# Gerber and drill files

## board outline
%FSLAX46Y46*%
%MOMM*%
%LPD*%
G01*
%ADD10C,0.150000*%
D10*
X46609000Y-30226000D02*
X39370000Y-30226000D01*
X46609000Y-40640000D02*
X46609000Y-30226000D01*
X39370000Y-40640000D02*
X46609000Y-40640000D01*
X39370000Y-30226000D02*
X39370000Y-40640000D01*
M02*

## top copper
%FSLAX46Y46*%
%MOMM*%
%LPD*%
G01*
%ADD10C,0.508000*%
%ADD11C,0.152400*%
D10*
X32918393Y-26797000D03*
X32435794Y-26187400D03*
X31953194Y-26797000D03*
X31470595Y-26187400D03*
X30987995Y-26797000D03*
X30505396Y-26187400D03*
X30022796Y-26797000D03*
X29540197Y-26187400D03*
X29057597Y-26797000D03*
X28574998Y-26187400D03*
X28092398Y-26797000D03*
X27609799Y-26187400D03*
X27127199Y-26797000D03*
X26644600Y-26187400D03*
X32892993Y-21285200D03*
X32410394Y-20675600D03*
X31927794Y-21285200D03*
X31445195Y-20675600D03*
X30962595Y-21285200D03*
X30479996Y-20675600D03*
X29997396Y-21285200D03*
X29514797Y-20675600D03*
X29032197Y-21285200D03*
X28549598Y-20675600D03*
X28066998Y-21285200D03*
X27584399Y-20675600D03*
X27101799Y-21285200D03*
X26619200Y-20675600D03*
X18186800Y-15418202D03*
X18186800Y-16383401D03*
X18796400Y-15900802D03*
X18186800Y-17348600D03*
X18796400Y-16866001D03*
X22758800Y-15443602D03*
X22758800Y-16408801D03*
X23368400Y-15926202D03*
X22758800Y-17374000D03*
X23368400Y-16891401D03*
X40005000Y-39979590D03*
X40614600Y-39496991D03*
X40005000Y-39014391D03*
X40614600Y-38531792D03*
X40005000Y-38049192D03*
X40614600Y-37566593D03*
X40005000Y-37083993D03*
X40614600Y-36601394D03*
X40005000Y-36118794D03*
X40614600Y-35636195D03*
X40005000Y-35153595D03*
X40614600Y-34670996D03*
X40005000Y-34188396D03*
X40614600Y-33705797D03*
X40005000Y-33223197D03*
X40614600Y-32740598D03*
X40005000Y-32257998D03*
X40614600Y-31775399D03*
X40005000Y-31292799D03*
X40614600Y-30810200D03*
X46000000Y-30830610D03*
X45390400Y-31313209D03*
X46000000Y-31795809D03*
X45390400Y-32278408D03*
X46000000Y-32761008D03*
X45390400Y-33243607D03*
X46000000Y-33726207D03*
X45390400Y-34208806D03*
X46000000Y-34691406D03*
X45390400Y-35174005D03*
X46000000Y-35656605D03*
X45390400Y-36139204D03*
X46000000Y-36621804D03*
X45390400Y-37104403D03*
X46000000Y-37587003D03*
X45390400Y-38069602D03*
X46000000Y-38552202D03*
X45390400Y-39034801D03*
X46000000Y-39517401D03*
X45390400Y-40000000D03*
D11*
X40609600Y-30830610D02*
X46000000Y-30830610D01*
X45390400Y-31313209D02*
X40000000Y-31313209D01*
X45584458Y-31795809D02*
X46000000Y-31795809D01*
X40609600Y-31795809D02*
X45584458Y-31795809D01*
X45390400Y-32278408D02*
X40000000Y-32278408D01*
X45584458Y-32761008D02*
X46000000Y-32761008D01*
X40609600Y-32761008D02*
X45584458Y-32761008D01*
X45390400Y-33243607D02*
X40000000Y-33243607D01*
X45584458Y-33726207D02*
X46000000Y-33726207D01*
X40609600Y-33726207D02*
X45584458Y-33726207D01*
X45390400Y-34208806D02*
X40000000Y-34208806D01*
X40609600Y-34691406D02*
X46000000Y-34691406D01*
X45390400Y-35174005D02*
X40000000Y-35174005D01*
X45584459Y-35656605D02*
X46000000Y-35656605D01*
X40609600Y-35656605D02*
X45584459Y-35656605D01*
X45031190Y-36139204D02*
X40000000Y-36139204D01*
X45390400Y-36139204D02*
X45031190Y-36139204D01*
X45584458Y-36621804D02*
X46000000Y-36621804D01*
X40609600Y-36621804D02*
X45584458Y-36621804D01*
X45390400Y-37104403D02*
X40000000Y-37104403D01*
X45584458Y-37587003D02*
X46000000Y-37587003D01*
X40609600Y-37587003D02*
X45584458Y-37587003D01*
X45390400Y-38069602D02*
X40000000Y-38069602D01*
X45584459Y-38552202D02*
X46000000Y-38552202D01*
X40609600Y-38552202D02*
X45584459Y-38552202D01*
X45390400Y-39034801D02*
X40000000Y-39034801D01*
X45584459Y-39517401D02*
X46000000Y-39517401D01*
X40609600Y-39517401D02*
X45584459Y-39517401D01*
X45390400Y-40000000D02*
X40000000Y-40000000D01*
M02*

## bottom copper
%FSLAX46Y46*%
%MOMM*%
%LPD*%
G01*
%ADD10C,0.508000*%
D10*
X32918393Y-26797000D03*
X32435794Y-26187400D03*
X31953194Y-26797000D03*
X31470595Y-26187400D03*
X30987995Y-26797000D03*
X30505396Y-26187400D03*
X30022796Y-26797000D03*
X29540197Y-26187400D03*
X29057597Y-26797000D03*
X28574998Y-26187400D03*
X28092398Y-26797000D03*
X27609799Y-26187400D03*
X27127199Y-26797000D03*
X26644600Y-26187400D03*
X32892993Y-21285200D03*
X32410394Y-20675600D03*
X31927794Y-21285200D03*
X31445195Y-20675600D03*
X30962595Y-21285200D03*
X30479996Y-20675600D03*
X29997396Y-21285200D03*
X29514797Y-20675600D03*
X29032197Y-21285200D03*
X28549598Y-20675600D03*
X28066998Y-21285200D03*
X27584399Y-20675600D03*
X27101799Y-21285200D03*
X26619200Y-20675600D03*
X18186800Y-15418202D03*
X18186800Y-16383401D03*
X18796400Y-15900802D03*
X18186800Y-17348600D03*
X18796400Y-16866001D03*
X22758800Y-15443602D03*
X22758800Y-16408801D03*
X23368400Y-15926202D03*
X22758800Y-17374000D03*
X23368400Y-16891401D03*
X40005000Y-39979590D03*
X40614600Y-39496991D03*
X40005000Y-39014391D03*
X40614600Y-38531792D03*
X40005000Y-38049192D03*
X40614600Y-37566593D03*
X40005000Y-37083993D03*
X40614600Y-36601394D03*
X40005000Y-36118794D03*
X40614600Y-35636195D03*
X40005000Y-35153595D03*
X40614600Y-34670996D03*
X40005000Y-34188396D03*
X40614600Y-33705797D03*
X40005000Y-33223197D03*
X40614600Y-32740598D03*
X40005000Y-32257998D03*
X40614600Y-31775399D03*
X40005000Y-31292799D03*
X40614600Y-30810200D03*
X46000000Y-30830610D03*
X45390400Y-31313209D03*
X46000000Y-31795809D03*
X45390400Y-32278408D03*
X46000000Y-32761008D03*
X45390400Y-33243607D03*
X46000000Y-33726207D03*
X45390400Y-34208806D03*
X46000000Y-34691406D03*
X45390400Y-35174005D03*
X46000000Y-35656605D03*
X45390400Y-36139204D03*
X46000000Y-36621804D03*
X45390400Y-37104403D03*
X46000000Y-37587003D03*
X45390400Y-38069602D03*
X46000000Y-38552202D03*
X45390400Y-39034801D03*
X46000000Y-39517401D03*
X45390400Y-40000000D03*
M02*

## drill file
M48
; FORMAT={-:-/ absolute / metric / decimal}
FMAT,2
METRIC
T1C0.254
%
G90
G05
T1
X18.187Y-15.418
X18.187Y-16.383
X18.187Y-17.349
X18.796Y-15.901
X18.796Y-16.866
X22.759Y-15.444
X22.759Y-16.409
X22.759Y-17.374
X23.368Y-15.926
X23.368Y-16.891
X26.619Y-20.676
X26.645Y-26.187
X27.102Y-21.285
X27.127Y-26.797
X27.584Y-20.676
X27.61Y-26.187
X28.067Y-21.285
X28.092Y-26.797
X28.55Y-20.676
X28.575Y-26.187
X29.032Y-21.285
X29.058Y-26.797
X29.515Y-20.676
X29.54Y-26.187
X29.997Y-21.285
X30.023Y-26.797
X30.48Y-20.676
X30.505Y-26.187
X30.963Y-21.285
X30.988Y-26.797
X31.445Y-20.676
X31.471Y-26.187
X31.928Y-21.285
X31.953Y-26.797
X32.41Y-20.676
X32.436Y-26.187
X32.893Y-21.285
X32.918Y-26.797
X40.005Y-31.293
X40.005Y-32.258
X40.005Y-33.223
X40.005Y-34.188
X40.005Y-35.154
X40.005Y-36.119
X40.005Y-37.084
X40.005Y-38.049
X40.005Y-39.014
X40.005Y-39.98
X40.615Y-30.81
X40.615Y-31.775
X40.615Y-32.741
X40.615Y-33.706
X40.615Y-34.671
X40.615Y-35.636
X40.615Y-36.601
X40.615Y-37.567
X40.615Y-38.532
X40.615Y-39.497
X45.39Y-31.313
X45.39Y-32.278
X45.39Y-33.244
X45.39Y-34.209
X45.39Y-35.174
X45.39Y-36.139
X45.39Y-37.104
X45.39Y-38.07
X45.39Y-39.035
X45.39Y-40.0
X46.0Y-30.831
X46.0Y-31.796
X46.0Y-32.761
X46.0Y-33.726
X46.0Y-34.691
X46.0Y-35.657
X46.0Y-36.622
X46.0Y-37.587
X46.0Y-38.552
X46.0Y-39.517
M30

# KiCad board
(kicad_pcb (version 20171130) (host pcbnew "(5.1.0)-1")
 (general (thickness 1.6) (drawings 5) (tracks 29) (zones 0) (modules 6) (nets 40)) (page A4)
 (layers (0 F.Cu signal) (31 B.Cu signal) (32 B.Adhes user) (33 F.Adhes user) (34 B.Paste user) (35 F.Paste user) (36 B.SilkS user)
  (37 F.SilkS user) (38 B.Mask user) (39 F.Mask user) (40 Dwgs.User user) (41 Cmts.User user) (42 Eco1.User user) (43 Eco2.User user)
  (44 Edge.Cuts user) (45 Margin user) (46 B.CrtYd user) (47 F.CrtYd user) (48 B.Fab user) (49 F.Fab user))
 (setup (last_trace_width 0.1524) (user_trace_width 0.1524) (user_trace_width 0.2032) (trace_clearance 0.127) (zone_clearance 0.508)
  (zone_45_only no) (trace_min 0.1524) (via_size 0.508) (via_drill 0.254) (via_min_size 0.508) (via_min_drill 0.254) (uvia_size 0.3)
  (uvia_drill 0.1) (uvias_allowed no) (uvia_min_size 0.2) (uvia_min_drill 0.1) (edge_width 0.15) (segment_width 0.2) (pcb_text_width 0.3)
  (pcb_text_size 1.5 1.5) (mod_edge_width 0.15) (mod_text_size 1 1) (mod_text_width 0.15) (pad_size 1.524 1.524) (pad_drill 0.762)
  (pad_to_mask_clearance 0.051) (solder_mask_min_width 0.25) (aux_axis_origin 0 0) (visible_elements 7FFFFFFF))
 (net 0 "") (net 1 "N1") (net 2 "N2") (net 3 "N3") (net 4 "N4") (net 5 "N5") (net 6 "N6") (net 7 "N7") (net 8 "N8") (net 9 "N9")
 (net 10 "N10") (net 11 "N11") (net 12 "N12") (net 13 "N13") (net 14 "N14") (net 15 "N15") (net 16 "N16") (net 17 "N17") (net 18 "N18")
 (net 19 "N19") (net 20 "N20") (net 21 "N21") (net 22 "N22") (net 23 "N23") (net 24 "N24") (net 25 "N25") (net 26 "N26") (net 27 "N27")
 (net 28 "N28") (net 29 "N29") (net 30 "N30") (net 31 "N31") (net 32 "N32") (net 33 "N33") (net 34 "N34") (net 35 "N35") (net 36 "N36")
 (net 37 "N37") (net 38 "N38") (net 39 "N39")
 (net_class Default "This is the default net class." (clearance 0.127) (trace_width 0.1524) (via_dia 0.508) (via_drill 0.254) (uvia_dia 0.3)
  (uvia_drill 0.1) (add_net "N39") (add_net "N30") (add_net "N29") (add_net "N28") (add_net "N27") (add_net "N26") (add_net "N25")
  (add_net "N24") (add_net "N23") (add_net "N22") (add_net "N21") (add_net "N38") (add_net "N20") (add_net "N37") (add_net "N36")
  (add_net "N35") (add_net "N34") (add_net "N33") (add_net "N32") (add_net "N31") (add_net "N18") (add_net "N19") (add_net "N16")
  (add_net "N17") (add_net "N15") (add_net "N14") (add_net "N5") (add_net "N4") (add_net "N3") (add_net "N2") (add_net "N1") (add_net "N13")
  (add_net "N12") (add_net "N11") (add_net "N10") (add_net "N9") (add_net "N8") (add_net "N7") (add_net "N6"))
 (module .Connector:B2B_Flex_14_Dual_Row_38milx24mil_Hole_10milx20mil (layer F.Cu) (at 26.6446 26.1874)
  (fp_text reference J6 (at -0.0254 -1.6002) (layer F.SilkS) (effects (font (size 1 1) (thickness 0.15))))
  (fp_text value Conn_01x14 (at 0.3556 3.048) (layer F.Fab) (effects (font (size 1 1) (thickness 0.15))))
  (pad 14 thru_hole circle (at 6.273793 0.6096) (size 0.508 0.508) (drill 0.254) (layers *.Cu *.Mask) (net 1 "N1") (zone_connect 0))
  (pad 13 thru_hole circle (at 5.791194 0) (size 0.508 0.508) (drill 0.254) (layers *.Cu *.Mask) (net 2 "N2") (zone_connect 0))
  (pad 12 thru_hole circle (at 5.308594 0.6096) (size 0.508 0.508) (drill 0.254) (layers *.Cu *.Mask) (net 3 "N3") (zone_connect 0))
  (pad 11 thru_hole circle (at 4.825995 0) (size 0.508 0.508) (drill 0.254) (layers *.Cu *.Mask) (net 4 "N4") (zone_connect 0))
  (pad 10 thru_hole circle (at 4.343395 0.6096) (size 0.508 0.508) (drill 0.254) (layers *.Cu *.Mask) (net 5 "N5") (zone_connect 0))
  (pad 9 thru_hole circle (at 3.860796 0) (size 0.508 0.508) (drill 0.254) (layers *.Cu *.Mask) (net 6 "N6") (zone_connect 0))
  (pad 8 thru_hole circle (at 3.378196 0.6096) (size 0.508 0.508) (drill 0.254) (layers *.Cu *.Mask) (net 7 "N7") (zone_connect 0))
  (pad 7 thru_hole circle (at 2.895597 0) (size 0.508 0.508) (drill 0.254) (layers *.Cu *.Mask) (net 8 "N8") (zone_connect 0))
  (pad 6 thru_hole circle (at 2.412997 0.6096) (size 0.508 0.508) (drill 0.254) (layers *.Cu *.Mask) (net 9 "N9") (zone_connect 0))
  (pad 5 thru_hole circle (at 1.930398 0) (size 0.508 0.508) (drill 0.254) (layers *.Cu *.Mask) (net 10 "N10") (zone_connect 0))
  (pad 4 thru_hole circle (at 1.447798 0.6096) (size 0.508 0.508) (drill 0.254) (layers *.Cu *.Mask) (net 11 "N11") (zone_connect 0))
  (pad 3 thru_hole circle (at 0.965199 0) (size 0.508 0.508) (drill 0.254) (layers *.Cu *.Mask) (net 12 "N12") (zone_connect 0))
  (pad 2 thru_hole circle (at 0.482599 0.6096) (size 0.508 0.508) (drill 0.254) (layers *.Cu *.Mask) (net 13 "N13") (zone_connect 0))
  (pad 1 thru_hole circle (at 0 0) (size 0.508 0.508) (drill 0.254) (layers *.Cu *.Mask) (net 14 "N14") (zone_connect 0)))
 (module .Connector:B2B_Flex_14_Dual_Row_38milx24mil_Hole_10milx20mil (layer F.Cu) (at 26.6192 20.6756)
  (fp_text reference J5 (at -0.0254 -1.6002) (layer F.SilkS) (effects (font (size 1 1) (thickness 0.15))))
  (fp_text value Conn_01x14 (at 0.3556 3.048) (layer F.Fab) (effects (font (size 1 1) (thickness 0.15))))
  (pad 14 thru_hole circle (at 6.273793 0.6096) (size 0.508 0.508) (drill 0.254) (layers *.Cu *.Mask) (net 1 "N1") (zone_connect 0))
  (pad 13 thru_hole circle (at 5.791194 0) (size 0.508 0.508) (drill 0.254) (layers *.Cu *.Mask) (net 2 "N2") (zone_connect 0))
  (pad 12 thru_hole circle (at 5.308594 0.6096) (size 0.508 0.508) (drill 0.254) (layers *.Cu *.Mask) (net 3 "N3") (zone_connect 0))
  (pad 11 thru_hole circle (at 4.825995 0) (size 0.508 0.508) (drill 0.254) (layers *.Cu *.Mask) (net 4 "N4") (zone_connect 0))
  (pad 10 thru_hole circle (at 4.343395 0.6096) (size 0.508 0.508) (drill 0.254) (layers *.Cu *.Mask) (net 5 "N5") (zone_connect 0))
  (pad 9 thru_hole circle (at 3.860796 0) (size 0.508 0.508) (drill 0.254) (layers *.Cu *.Mask) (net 6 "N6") (zone_connect 0))
  (pad 8 thru_hole circle (at 3.378196 0.6096) (size 0.508 0.508) (drill 0.254) (layers *.Cu *.Mask) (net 7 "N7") (zone_connect 0))
  (pad 7 thru_hole circle (at 2.895597 0) (size 0.508 0.508) (drill 0.254) (layers *.Cu *.Mask) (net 8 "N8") (zone_connect 0))
  (pad 6 thru_hole circle (at 2.412997 0.6096) (size 0.508 0.508) (drill 0.254) (layers *.Cu *.Mask) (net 9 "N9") (zone_connect 0))
  (pad 5 thru_hole circle (at 1.930398 0) (size 0.508 0.508) (drill 0.254) (layers *.Cu *.Mask) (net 10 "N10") (zone_connect 0))
  (pad 4 thru_hole circle (at 1.447798 0.6096) (size 0.508 0.508) (drill 0.254) (layers *.Cu *.Mask) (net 11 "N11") (zone_connect 0))
  (pad 3 thru_hole circle (at 0.965199 0) (size 0.508 0.508) (drill 0.254) (layers *.Cu *.Mask) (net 12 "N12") (zone_connect 0))
  (pad 2 thru_hole circle (at 0.482599 0.6096) (size 0.508 0.508) (drill 0.254) (layers *.Cu *.Mask) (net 13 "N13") (zone_connect 0))
  (pad 1 thru_hole circle (at 0 0) (size 0.508 0.508) (drill 0.254) (layers *.Cu *.Mask) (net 14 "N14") (zone_connect 0)))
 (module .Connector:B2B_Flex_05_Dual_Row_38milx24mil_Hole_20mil (layer F.Cu) (at 18.2118 17.3736 90)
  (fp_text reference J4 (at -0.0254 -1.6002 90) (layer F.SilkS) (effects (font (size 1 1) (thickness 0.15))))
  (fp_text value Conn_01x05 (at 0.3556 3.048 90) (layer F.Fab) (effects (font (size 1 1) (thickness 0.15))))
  (pad 5 thru_hole circle (at 1.955398 -0.025 90) (size 0.508 0.508) (drill 0.254) (layers *.Cu *.Mask) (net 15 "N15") (zone_connect 0))
  (pad 3 thru_hole circle (at 0.990199 -0.025 90) (size 0.508 0.508) (drill 0.254) (layers *.Cu *.Mask) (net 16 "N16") (zone_connect 0))
  (pad 4 thru_hole circle (at 1.472798 0.5846 90) (size 0.508 0.508) (drill 0.254) (layers *.Cu *.Mask) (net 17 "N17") (zone_connect 0))
  (pad 1 thru_hole circle (at 0.025 -0.025 90) (size 0.508 0.508) (drill 0.254) (layers *.Cu *.Mask) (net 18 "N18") (zone_connect 0))
  (pad 2 thru_hole circle (at 0.507599 0.5846 90) (size 0.508 0.508) (drill 0.254) (layers *.Cu *.Mask) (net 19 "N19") (zone_connect 0)))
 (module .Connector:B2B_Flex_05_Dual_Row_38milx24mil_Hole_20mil (layer F.Cu) (at 22.7838 17.399 90)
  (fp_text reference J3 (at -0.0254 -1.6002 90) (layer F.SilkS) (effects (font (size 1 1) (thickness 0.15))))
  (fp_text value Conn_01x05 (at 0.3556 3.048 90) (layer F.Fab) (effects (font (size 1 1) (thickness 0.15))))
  (pad 5 thru_hole circle (at 1.955398 -0.025 90) (size 0.508 0.508) (drill 0.254) (layers *.Cu *.Mask) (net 15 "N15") (zone_connect 0))
  (pad 3 thru_hole circle (at 0.990199 -0.025 90) (size 0.508 0.508) (drill 0.254) (layers *.Cu *.Mask) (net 16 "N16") (zone_connect 0))
  (pad 4 thru_hole circle (at 1.472798 0.5846 90) (size 0.508 0.508) (drill 0.254) (layers *.Cu *.Mask) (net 17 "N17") (zone_connect 0))
  (pad 1 thru_hole circle (at 0.025 -0.025 90) (size 0.508 0.508) (drill 0.254) (layers *.Cu *.Mask) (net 18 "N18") (zone_connect 0))
  (pad 2 thru_hole circle (at 0.507599 0.5846 90) (size 0.508 0.508) (drill 0.254) (layers *.Cu *.Mask) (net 19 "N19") (zone_connect 0)))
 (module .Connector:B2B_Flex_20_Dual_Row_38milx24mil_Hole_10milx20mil (layer F.Cu) (at 40.6146 30.8102 270)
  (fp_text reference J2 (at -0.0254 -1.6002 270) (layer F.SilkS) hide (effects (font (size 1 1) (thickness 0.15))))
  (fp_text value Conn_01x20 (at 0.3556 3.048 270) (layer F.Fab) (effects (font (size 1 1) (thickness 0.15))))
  (pad 20 thru_hole circle (at 9.16939 0.6096 270) (size 0.508 0.508) (drill 0.254) (layers *.Cu *.Mask) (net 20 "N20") (zone_connect 0))
  (pad 19 thru_hole circle (at 8.686791 0 270) (size 0.508 0.508) (drill 0.254) (layers *.Cu *.Mask) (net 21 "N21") (zone_connect 0))
  (pad 18 thru_hole circle (at 8.204191 0.6096 270) (size 0.508 0.508) (drill 0.254) (layers *.Cu *.Mask) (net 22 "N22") (zone_connect 0))
  (pad 17 thru_hole circle (at 7.721592 0 270) (size 0.508 0.508) (drill 0.254) (layers *.Cu *.Mask) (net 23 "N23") (zone_connect 0))
  (pad 16 thru_hole circle (at 7.238992 0.6096 270) (size 0.508 0.508) (drill 0.254) (layers *.Cu *.Mask) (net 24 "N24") (zone_connect 0))
  (pad 15 thru_hole circle (at 6.756393 0 270) (size 0.508 0.508) (drill 0.254) (layers *.Cu *.Mask) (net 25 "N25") (zone_connect 0))
  (pad 14 thru_hole circle (at 6.273793 0.6096 270) (size 0.508 0.508) (drill 0.254) (layers *.Cu *.Mask) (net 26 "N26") (zone_connect 0))
  (pad 13 thru_hole circle (at 5.791194 0 270) (size 0.508 0.508) (drill 0.254) (layers *.Cu *.Mask) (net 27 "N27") (zone_connect 0))
  (pad 12 thru_hole circle (at 5.308594 0.6096 270) (size 0.508 0.508) (drill 0.254) (layers *.Cu *.Mask) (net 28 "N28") (zone_connect 0))
  (pad 11 thru_hole circle (at 4.825995 0 270) (size 0.508 0.508) (drill 0.254) (layers *.Cu *.Mask) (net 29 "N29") (zone_connect 0))
  (pad 10 thru_hole circle (at 4.343395 0.6096 270) (size 0.508 0.508) (drill 0.254) (layers *.Cu *.Mask) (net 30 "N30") (zone_connect 0))
  (pad 9 thru_hole circle (at 3.860796 0 270) (size 0.508 0.508) (drill 0.254) (layers *.Cu *.Mask) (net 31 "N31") (zone_connect 0))
  (pad 8 thru_hole circle (at 3.378196 0.6096 270) (size 0.508 0.508) (drill 0.254) (layers *.Cu *.Mask) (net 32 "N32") (zone_connect 0))
  (pad 7 thru_hole circle (at 2.895597 0 270) (size 0.508 0.508) (drill 0.254) (layers *.Cu *.Mask) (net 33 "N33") (zone_connect 0))
  (pad 6 thru_hole circle (at 2.412997 0.6096 270) (size 0.508 0.508) (drill 0.254) (layers *.Cu *.Mask) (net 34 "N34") (zone_connect 0))
  (pad 5 thru_hole circle (at 1.930398 0 270) (size 0.508 0.508) (drill 0.254) (layers *.Cu *.Mask) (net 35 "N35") (zone_connect 0))
  (pad 4 thru_hole circle (at 1.447798 0.6096 270) (size 0.508 0.508) (drill 0.254) (layers *.Cu *.Mask) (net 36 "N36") (zone_connect 0))
  (pad 3 thru_hole circle (at 0.965199 0 270) (size 0.508 0.508) (drill 0.254) (layers *.Cu *.Mask) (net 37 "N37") (zone_connect 0))
  (pad 2 thru_hole circle (at 0.482599 0.6096 270) (size 0.508 0.508) (drill 0.254) (layers *.Cu *.Mask) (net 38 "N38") (zone_connect 0))
  (pad 1 thru_hole circle (at 0 0 270) (size 0.508 0.508) (drill 0.254) (layers *.Cu *.Mask) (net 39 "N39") (zone_connect 0)))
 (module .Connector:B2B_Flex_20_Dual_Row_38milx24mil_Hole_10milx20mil (layer F.Cu) (at 46 30.83061 270)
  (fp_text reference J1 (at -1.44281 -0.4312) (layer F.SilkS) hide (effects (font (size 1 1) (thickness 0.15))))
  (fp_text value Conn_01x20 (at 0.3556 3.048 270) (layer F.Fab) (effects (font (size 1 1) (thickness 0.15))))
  (pad 1 thru_hole circle (at 0 0 270) (size 0.508 0.508) (drill 0.254) (layers *.Cu *.Mask) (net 39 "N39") (zone_connect 0))
  (pad 2 thru_hole circle (at 0.482599 0.6096 270) (size 0.508 0.508) (drill 0.254) (layers *.Cu *.Mask) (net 38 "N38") (zone_connect 0))
  (pad 3 thru_hole circle (at 0.965199 0 270) (size 0.508 0.508) (drill 0.254) (layers *.Cu *.Mask) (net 37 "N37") (zone_connect 0))
  (pad 4 thru_hole circle (at 1.447798 0.6096 270) (size 0.508 0.508) (drill 0.254) (layers *.Cu *.Mask) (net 36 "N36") (zone_connect 0))
  (pad 5 thru_hole circle (at 1.930398 0 270) (size 0.508 0.508) (drill 0.254) (layers *.Cu *.Mask) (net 35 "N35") (zone_connect 0))
  (pad 6 thru_hole circle (at 2.412997 0.6096 270) (size 0.508 0.508) (drill 0.254) (layers *.Cu *.Mask) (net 34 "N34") (zone_connect 0))
  (pad 7 thru_hole circle (at 2.895597 0 270) (size 0.508 0.508) (drill 0.254) (layers *.Cu *.Mask) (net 33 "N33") (zone_connect 0))
  (pad 8 thru_hole circle (at 3.378196 0.6096 270) (size 0.508 0.508) (drill 0.254) (layers *.Cu *.Mask) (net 32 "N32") (zone_connect 0))
  (pad 9 thru_hole circle (at 3.860796 0 270) (size 0.508 0.508) (drill 0.254) (layers *.Cu *.Mask) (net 31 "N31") (zone_connect 0))
  (pad 10 thru_hole circle (at 4.343395 0.6096 270) (size 0.508 0.508) (drill 0.254) (layers *.Cu *.Mask) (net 30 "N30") (zone_connect 0))
  (pad 11 thru_hole circle (at 4.825995 0 270) (size 0.508 0.508) (drill 0.254) (layers *.Cu *.Mask) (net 29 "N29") (zone_connect 0))
  (pad 12 thru_hole circle (at 5.308594 0.6096 270) (size 0.508 0.508) (drill 0.254) (layers *.Cu *.Mask) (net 28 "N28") (zone_connect 0))
  (pad 13 thru_hole circle (at 5.791194 0 270) (size 0.508 0.508) (drill 0.254) (layers *.Cu *.Mask) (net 27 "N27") (zone_connect 0))
  (pad 14 thru_hole circle (at 6.273793 0.6096 270) (size 0.508 0.508) (drill 0.254) (layers *.Cu *.Mask) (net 26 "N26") (zone_connect 0))
  (pad 15 thru_hole circle (at 6.756393 0 270) (size 0.508 0.508) (drill 0.254) (layers *.Cu *.Mask) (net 25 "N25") (zone_connect 0))
  (pad 16 thru_hole circle (at 7.238992 0.6096 270) (size 0.508 0.508) (drill 0.254) (layers *.Cu *.Mask) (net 24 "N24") (zone_connect 0))
  (pad 17 thru_hole circle (at 7.721592 0 270) (size 0.508 0.508) (drill 0.254) (layers *.Cu *.Mask) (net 23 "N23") (zone_connect 0))
  (pad 18 thru_hole circle (at 8.204191 0.6096 270) (size 0.508 0.508) (drill 0.254) (layers *.Cu *.Mask) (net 22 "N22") (zone_connect 0))
  (pad 19 thru_hole circle (at 8.686791 0 270) (size 0.508 0.508) (drill 0.254) (layers *.Cu *.Mask) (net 21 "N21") (zone_connect 0))
  (pad 20 thru_hole circle (at 9.16939 0.6096 270) (size 0.508 0.508) (drill 0.254) (layers *.Cu *.Mask) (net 20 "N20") (zone_connect 0)))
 (gr_line (start 46.609 30.226) (end 39.37 30.226) (layer Edge.Cuts) (width 0.15))
 (gr_line (start 46.609 40.64) (end 46.609 30.226) (layer Edge.Cuts) (width 0.15))
 (gr_line (start 39.37 40.64) (end 46.609 40.64) (layer Edge.Cuts) (width 0.15))
 (gr_line (start 39.37 30.226) (end 39.37 40.64) (layer Edge.Cuts) (width 0.15))
 (segment (start 40.6096 30.83061) (end 46 30.83061) (width 0.1524) (layer F.Cu) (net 39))
 (segment (start 45.3904 31.313209) (end 40 31.313209) (width 0.1524) (layer F.Cu) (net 38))
 (segment (start 45.584458 31.795809) (end 46 31.795809) (width 0.1524) (layer F.Cu) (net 37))
 (segment (start 40.6096 31.795809) (end 45.584458 31.795809) (width 0.1524) (layer F.Cu) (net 37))
 (segment (start 45.3904 32.278408) (end 40 32.278408) (width 0.1524) (layer F.Cu) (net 36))
 (segment (start 45.584458 32.761008) (end 46 32.761008) (width 0.1524) (layer F.Cu) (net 35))
 (segment (start 40.6096 32.761008) (end 45.584458 32.761008) (width 0.1524) (layer F.Cu) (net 35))
 (segment (start 45.3904 33.243607) (end 40 33.243607) (width 0.1524) (layer F.Cu) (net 34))
 (segment (start 45.584458 33.726207) (end 46 33.726207) (width 0.1524) (layer F.Cu) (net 33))
 (segment (start 40.6096 33.726207) (end 45.584458 33.726207) (width 0.1524) (layer F.Cu) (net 33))
 (segment (start 45.3904 34.208806) (end 40 34.208806) (width 0.1524) (layer F.Cu) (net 32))
 (segment (start 40.6096 34.691406) (end 46 34.691406) (width 0.1524) (layer F.Cu) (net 31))
 (segment (start 45.3904 35.174005) (end 40 35.174005) (width 0.1524) (layer F.Cu) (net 30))
 (segment (start 45.584459 35.656605) (end 46 35.656605) (width 0.1524) (layer F.Cu) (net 29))
 (segment (start 40.6096 35.656605) (end 45.584459 35.656605) (width 0.1524) (layer F.Cu) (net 29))
 (segment (start 45.03119 36.139204) (end 40 36.139204) (width 0.1524) (layer F.Cu) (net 28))
 (segment (start 45.3904 36.139204) (end 45.03119 36.139204) (width 0.1524) (layer F.Cu) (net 28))
 (segment (start 45.584458 36.621804) (end 46 36.621804) (width 0.1524) (layer F.Cu) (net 27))
 (segment (start 40.6096 36.621804) (end 45.584458 36.621804) (width 0.1524) (layer F.Cu) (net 27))
 (segment (start 45.3904 37.104403) (end 40 37.104403) (width 0.1524) (layer F.Cu) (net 26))
 (segment (start 45.584458 37.587003) (end 46 37.587003) (width 0.1524) (layer F.Cu) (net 25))
 (segment (start 40.6096 37.587003) (end 45.584458 37.587003) (width 0.1524) (layer F.Cu) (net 25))
 (segment (start 45.3904 38.069602) (end 40 38.069602) (width 0.1524) (layer F.Cu) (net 24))
 (segment (start 45.584459 38.552202) (end 46 38.552202) (width 0.1524) (layer F.Cu) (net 23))
 (segment (start 40.6096 38.552202) (end 45.584459 38.552202) (width 0.1524) (layer F.Cu) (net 23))
 (segment (start 45.3904 39.034801) (end 40 39.034801) (width 0.1524) (layer F.Cu) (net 22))
 (segment (start 45.584459 39.517401) (end 46 39.517401) (width 0.1524) (layer F.Cu) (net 21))
 (segment (start 40.6096 39.517401) (end 45.584459 39.517401) (width 0.1524) (layer F.Cu) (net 21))
 (segment (start 45.3904 40) (end 40 40) (width 0.1524) (layer F.Cu) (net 20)))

